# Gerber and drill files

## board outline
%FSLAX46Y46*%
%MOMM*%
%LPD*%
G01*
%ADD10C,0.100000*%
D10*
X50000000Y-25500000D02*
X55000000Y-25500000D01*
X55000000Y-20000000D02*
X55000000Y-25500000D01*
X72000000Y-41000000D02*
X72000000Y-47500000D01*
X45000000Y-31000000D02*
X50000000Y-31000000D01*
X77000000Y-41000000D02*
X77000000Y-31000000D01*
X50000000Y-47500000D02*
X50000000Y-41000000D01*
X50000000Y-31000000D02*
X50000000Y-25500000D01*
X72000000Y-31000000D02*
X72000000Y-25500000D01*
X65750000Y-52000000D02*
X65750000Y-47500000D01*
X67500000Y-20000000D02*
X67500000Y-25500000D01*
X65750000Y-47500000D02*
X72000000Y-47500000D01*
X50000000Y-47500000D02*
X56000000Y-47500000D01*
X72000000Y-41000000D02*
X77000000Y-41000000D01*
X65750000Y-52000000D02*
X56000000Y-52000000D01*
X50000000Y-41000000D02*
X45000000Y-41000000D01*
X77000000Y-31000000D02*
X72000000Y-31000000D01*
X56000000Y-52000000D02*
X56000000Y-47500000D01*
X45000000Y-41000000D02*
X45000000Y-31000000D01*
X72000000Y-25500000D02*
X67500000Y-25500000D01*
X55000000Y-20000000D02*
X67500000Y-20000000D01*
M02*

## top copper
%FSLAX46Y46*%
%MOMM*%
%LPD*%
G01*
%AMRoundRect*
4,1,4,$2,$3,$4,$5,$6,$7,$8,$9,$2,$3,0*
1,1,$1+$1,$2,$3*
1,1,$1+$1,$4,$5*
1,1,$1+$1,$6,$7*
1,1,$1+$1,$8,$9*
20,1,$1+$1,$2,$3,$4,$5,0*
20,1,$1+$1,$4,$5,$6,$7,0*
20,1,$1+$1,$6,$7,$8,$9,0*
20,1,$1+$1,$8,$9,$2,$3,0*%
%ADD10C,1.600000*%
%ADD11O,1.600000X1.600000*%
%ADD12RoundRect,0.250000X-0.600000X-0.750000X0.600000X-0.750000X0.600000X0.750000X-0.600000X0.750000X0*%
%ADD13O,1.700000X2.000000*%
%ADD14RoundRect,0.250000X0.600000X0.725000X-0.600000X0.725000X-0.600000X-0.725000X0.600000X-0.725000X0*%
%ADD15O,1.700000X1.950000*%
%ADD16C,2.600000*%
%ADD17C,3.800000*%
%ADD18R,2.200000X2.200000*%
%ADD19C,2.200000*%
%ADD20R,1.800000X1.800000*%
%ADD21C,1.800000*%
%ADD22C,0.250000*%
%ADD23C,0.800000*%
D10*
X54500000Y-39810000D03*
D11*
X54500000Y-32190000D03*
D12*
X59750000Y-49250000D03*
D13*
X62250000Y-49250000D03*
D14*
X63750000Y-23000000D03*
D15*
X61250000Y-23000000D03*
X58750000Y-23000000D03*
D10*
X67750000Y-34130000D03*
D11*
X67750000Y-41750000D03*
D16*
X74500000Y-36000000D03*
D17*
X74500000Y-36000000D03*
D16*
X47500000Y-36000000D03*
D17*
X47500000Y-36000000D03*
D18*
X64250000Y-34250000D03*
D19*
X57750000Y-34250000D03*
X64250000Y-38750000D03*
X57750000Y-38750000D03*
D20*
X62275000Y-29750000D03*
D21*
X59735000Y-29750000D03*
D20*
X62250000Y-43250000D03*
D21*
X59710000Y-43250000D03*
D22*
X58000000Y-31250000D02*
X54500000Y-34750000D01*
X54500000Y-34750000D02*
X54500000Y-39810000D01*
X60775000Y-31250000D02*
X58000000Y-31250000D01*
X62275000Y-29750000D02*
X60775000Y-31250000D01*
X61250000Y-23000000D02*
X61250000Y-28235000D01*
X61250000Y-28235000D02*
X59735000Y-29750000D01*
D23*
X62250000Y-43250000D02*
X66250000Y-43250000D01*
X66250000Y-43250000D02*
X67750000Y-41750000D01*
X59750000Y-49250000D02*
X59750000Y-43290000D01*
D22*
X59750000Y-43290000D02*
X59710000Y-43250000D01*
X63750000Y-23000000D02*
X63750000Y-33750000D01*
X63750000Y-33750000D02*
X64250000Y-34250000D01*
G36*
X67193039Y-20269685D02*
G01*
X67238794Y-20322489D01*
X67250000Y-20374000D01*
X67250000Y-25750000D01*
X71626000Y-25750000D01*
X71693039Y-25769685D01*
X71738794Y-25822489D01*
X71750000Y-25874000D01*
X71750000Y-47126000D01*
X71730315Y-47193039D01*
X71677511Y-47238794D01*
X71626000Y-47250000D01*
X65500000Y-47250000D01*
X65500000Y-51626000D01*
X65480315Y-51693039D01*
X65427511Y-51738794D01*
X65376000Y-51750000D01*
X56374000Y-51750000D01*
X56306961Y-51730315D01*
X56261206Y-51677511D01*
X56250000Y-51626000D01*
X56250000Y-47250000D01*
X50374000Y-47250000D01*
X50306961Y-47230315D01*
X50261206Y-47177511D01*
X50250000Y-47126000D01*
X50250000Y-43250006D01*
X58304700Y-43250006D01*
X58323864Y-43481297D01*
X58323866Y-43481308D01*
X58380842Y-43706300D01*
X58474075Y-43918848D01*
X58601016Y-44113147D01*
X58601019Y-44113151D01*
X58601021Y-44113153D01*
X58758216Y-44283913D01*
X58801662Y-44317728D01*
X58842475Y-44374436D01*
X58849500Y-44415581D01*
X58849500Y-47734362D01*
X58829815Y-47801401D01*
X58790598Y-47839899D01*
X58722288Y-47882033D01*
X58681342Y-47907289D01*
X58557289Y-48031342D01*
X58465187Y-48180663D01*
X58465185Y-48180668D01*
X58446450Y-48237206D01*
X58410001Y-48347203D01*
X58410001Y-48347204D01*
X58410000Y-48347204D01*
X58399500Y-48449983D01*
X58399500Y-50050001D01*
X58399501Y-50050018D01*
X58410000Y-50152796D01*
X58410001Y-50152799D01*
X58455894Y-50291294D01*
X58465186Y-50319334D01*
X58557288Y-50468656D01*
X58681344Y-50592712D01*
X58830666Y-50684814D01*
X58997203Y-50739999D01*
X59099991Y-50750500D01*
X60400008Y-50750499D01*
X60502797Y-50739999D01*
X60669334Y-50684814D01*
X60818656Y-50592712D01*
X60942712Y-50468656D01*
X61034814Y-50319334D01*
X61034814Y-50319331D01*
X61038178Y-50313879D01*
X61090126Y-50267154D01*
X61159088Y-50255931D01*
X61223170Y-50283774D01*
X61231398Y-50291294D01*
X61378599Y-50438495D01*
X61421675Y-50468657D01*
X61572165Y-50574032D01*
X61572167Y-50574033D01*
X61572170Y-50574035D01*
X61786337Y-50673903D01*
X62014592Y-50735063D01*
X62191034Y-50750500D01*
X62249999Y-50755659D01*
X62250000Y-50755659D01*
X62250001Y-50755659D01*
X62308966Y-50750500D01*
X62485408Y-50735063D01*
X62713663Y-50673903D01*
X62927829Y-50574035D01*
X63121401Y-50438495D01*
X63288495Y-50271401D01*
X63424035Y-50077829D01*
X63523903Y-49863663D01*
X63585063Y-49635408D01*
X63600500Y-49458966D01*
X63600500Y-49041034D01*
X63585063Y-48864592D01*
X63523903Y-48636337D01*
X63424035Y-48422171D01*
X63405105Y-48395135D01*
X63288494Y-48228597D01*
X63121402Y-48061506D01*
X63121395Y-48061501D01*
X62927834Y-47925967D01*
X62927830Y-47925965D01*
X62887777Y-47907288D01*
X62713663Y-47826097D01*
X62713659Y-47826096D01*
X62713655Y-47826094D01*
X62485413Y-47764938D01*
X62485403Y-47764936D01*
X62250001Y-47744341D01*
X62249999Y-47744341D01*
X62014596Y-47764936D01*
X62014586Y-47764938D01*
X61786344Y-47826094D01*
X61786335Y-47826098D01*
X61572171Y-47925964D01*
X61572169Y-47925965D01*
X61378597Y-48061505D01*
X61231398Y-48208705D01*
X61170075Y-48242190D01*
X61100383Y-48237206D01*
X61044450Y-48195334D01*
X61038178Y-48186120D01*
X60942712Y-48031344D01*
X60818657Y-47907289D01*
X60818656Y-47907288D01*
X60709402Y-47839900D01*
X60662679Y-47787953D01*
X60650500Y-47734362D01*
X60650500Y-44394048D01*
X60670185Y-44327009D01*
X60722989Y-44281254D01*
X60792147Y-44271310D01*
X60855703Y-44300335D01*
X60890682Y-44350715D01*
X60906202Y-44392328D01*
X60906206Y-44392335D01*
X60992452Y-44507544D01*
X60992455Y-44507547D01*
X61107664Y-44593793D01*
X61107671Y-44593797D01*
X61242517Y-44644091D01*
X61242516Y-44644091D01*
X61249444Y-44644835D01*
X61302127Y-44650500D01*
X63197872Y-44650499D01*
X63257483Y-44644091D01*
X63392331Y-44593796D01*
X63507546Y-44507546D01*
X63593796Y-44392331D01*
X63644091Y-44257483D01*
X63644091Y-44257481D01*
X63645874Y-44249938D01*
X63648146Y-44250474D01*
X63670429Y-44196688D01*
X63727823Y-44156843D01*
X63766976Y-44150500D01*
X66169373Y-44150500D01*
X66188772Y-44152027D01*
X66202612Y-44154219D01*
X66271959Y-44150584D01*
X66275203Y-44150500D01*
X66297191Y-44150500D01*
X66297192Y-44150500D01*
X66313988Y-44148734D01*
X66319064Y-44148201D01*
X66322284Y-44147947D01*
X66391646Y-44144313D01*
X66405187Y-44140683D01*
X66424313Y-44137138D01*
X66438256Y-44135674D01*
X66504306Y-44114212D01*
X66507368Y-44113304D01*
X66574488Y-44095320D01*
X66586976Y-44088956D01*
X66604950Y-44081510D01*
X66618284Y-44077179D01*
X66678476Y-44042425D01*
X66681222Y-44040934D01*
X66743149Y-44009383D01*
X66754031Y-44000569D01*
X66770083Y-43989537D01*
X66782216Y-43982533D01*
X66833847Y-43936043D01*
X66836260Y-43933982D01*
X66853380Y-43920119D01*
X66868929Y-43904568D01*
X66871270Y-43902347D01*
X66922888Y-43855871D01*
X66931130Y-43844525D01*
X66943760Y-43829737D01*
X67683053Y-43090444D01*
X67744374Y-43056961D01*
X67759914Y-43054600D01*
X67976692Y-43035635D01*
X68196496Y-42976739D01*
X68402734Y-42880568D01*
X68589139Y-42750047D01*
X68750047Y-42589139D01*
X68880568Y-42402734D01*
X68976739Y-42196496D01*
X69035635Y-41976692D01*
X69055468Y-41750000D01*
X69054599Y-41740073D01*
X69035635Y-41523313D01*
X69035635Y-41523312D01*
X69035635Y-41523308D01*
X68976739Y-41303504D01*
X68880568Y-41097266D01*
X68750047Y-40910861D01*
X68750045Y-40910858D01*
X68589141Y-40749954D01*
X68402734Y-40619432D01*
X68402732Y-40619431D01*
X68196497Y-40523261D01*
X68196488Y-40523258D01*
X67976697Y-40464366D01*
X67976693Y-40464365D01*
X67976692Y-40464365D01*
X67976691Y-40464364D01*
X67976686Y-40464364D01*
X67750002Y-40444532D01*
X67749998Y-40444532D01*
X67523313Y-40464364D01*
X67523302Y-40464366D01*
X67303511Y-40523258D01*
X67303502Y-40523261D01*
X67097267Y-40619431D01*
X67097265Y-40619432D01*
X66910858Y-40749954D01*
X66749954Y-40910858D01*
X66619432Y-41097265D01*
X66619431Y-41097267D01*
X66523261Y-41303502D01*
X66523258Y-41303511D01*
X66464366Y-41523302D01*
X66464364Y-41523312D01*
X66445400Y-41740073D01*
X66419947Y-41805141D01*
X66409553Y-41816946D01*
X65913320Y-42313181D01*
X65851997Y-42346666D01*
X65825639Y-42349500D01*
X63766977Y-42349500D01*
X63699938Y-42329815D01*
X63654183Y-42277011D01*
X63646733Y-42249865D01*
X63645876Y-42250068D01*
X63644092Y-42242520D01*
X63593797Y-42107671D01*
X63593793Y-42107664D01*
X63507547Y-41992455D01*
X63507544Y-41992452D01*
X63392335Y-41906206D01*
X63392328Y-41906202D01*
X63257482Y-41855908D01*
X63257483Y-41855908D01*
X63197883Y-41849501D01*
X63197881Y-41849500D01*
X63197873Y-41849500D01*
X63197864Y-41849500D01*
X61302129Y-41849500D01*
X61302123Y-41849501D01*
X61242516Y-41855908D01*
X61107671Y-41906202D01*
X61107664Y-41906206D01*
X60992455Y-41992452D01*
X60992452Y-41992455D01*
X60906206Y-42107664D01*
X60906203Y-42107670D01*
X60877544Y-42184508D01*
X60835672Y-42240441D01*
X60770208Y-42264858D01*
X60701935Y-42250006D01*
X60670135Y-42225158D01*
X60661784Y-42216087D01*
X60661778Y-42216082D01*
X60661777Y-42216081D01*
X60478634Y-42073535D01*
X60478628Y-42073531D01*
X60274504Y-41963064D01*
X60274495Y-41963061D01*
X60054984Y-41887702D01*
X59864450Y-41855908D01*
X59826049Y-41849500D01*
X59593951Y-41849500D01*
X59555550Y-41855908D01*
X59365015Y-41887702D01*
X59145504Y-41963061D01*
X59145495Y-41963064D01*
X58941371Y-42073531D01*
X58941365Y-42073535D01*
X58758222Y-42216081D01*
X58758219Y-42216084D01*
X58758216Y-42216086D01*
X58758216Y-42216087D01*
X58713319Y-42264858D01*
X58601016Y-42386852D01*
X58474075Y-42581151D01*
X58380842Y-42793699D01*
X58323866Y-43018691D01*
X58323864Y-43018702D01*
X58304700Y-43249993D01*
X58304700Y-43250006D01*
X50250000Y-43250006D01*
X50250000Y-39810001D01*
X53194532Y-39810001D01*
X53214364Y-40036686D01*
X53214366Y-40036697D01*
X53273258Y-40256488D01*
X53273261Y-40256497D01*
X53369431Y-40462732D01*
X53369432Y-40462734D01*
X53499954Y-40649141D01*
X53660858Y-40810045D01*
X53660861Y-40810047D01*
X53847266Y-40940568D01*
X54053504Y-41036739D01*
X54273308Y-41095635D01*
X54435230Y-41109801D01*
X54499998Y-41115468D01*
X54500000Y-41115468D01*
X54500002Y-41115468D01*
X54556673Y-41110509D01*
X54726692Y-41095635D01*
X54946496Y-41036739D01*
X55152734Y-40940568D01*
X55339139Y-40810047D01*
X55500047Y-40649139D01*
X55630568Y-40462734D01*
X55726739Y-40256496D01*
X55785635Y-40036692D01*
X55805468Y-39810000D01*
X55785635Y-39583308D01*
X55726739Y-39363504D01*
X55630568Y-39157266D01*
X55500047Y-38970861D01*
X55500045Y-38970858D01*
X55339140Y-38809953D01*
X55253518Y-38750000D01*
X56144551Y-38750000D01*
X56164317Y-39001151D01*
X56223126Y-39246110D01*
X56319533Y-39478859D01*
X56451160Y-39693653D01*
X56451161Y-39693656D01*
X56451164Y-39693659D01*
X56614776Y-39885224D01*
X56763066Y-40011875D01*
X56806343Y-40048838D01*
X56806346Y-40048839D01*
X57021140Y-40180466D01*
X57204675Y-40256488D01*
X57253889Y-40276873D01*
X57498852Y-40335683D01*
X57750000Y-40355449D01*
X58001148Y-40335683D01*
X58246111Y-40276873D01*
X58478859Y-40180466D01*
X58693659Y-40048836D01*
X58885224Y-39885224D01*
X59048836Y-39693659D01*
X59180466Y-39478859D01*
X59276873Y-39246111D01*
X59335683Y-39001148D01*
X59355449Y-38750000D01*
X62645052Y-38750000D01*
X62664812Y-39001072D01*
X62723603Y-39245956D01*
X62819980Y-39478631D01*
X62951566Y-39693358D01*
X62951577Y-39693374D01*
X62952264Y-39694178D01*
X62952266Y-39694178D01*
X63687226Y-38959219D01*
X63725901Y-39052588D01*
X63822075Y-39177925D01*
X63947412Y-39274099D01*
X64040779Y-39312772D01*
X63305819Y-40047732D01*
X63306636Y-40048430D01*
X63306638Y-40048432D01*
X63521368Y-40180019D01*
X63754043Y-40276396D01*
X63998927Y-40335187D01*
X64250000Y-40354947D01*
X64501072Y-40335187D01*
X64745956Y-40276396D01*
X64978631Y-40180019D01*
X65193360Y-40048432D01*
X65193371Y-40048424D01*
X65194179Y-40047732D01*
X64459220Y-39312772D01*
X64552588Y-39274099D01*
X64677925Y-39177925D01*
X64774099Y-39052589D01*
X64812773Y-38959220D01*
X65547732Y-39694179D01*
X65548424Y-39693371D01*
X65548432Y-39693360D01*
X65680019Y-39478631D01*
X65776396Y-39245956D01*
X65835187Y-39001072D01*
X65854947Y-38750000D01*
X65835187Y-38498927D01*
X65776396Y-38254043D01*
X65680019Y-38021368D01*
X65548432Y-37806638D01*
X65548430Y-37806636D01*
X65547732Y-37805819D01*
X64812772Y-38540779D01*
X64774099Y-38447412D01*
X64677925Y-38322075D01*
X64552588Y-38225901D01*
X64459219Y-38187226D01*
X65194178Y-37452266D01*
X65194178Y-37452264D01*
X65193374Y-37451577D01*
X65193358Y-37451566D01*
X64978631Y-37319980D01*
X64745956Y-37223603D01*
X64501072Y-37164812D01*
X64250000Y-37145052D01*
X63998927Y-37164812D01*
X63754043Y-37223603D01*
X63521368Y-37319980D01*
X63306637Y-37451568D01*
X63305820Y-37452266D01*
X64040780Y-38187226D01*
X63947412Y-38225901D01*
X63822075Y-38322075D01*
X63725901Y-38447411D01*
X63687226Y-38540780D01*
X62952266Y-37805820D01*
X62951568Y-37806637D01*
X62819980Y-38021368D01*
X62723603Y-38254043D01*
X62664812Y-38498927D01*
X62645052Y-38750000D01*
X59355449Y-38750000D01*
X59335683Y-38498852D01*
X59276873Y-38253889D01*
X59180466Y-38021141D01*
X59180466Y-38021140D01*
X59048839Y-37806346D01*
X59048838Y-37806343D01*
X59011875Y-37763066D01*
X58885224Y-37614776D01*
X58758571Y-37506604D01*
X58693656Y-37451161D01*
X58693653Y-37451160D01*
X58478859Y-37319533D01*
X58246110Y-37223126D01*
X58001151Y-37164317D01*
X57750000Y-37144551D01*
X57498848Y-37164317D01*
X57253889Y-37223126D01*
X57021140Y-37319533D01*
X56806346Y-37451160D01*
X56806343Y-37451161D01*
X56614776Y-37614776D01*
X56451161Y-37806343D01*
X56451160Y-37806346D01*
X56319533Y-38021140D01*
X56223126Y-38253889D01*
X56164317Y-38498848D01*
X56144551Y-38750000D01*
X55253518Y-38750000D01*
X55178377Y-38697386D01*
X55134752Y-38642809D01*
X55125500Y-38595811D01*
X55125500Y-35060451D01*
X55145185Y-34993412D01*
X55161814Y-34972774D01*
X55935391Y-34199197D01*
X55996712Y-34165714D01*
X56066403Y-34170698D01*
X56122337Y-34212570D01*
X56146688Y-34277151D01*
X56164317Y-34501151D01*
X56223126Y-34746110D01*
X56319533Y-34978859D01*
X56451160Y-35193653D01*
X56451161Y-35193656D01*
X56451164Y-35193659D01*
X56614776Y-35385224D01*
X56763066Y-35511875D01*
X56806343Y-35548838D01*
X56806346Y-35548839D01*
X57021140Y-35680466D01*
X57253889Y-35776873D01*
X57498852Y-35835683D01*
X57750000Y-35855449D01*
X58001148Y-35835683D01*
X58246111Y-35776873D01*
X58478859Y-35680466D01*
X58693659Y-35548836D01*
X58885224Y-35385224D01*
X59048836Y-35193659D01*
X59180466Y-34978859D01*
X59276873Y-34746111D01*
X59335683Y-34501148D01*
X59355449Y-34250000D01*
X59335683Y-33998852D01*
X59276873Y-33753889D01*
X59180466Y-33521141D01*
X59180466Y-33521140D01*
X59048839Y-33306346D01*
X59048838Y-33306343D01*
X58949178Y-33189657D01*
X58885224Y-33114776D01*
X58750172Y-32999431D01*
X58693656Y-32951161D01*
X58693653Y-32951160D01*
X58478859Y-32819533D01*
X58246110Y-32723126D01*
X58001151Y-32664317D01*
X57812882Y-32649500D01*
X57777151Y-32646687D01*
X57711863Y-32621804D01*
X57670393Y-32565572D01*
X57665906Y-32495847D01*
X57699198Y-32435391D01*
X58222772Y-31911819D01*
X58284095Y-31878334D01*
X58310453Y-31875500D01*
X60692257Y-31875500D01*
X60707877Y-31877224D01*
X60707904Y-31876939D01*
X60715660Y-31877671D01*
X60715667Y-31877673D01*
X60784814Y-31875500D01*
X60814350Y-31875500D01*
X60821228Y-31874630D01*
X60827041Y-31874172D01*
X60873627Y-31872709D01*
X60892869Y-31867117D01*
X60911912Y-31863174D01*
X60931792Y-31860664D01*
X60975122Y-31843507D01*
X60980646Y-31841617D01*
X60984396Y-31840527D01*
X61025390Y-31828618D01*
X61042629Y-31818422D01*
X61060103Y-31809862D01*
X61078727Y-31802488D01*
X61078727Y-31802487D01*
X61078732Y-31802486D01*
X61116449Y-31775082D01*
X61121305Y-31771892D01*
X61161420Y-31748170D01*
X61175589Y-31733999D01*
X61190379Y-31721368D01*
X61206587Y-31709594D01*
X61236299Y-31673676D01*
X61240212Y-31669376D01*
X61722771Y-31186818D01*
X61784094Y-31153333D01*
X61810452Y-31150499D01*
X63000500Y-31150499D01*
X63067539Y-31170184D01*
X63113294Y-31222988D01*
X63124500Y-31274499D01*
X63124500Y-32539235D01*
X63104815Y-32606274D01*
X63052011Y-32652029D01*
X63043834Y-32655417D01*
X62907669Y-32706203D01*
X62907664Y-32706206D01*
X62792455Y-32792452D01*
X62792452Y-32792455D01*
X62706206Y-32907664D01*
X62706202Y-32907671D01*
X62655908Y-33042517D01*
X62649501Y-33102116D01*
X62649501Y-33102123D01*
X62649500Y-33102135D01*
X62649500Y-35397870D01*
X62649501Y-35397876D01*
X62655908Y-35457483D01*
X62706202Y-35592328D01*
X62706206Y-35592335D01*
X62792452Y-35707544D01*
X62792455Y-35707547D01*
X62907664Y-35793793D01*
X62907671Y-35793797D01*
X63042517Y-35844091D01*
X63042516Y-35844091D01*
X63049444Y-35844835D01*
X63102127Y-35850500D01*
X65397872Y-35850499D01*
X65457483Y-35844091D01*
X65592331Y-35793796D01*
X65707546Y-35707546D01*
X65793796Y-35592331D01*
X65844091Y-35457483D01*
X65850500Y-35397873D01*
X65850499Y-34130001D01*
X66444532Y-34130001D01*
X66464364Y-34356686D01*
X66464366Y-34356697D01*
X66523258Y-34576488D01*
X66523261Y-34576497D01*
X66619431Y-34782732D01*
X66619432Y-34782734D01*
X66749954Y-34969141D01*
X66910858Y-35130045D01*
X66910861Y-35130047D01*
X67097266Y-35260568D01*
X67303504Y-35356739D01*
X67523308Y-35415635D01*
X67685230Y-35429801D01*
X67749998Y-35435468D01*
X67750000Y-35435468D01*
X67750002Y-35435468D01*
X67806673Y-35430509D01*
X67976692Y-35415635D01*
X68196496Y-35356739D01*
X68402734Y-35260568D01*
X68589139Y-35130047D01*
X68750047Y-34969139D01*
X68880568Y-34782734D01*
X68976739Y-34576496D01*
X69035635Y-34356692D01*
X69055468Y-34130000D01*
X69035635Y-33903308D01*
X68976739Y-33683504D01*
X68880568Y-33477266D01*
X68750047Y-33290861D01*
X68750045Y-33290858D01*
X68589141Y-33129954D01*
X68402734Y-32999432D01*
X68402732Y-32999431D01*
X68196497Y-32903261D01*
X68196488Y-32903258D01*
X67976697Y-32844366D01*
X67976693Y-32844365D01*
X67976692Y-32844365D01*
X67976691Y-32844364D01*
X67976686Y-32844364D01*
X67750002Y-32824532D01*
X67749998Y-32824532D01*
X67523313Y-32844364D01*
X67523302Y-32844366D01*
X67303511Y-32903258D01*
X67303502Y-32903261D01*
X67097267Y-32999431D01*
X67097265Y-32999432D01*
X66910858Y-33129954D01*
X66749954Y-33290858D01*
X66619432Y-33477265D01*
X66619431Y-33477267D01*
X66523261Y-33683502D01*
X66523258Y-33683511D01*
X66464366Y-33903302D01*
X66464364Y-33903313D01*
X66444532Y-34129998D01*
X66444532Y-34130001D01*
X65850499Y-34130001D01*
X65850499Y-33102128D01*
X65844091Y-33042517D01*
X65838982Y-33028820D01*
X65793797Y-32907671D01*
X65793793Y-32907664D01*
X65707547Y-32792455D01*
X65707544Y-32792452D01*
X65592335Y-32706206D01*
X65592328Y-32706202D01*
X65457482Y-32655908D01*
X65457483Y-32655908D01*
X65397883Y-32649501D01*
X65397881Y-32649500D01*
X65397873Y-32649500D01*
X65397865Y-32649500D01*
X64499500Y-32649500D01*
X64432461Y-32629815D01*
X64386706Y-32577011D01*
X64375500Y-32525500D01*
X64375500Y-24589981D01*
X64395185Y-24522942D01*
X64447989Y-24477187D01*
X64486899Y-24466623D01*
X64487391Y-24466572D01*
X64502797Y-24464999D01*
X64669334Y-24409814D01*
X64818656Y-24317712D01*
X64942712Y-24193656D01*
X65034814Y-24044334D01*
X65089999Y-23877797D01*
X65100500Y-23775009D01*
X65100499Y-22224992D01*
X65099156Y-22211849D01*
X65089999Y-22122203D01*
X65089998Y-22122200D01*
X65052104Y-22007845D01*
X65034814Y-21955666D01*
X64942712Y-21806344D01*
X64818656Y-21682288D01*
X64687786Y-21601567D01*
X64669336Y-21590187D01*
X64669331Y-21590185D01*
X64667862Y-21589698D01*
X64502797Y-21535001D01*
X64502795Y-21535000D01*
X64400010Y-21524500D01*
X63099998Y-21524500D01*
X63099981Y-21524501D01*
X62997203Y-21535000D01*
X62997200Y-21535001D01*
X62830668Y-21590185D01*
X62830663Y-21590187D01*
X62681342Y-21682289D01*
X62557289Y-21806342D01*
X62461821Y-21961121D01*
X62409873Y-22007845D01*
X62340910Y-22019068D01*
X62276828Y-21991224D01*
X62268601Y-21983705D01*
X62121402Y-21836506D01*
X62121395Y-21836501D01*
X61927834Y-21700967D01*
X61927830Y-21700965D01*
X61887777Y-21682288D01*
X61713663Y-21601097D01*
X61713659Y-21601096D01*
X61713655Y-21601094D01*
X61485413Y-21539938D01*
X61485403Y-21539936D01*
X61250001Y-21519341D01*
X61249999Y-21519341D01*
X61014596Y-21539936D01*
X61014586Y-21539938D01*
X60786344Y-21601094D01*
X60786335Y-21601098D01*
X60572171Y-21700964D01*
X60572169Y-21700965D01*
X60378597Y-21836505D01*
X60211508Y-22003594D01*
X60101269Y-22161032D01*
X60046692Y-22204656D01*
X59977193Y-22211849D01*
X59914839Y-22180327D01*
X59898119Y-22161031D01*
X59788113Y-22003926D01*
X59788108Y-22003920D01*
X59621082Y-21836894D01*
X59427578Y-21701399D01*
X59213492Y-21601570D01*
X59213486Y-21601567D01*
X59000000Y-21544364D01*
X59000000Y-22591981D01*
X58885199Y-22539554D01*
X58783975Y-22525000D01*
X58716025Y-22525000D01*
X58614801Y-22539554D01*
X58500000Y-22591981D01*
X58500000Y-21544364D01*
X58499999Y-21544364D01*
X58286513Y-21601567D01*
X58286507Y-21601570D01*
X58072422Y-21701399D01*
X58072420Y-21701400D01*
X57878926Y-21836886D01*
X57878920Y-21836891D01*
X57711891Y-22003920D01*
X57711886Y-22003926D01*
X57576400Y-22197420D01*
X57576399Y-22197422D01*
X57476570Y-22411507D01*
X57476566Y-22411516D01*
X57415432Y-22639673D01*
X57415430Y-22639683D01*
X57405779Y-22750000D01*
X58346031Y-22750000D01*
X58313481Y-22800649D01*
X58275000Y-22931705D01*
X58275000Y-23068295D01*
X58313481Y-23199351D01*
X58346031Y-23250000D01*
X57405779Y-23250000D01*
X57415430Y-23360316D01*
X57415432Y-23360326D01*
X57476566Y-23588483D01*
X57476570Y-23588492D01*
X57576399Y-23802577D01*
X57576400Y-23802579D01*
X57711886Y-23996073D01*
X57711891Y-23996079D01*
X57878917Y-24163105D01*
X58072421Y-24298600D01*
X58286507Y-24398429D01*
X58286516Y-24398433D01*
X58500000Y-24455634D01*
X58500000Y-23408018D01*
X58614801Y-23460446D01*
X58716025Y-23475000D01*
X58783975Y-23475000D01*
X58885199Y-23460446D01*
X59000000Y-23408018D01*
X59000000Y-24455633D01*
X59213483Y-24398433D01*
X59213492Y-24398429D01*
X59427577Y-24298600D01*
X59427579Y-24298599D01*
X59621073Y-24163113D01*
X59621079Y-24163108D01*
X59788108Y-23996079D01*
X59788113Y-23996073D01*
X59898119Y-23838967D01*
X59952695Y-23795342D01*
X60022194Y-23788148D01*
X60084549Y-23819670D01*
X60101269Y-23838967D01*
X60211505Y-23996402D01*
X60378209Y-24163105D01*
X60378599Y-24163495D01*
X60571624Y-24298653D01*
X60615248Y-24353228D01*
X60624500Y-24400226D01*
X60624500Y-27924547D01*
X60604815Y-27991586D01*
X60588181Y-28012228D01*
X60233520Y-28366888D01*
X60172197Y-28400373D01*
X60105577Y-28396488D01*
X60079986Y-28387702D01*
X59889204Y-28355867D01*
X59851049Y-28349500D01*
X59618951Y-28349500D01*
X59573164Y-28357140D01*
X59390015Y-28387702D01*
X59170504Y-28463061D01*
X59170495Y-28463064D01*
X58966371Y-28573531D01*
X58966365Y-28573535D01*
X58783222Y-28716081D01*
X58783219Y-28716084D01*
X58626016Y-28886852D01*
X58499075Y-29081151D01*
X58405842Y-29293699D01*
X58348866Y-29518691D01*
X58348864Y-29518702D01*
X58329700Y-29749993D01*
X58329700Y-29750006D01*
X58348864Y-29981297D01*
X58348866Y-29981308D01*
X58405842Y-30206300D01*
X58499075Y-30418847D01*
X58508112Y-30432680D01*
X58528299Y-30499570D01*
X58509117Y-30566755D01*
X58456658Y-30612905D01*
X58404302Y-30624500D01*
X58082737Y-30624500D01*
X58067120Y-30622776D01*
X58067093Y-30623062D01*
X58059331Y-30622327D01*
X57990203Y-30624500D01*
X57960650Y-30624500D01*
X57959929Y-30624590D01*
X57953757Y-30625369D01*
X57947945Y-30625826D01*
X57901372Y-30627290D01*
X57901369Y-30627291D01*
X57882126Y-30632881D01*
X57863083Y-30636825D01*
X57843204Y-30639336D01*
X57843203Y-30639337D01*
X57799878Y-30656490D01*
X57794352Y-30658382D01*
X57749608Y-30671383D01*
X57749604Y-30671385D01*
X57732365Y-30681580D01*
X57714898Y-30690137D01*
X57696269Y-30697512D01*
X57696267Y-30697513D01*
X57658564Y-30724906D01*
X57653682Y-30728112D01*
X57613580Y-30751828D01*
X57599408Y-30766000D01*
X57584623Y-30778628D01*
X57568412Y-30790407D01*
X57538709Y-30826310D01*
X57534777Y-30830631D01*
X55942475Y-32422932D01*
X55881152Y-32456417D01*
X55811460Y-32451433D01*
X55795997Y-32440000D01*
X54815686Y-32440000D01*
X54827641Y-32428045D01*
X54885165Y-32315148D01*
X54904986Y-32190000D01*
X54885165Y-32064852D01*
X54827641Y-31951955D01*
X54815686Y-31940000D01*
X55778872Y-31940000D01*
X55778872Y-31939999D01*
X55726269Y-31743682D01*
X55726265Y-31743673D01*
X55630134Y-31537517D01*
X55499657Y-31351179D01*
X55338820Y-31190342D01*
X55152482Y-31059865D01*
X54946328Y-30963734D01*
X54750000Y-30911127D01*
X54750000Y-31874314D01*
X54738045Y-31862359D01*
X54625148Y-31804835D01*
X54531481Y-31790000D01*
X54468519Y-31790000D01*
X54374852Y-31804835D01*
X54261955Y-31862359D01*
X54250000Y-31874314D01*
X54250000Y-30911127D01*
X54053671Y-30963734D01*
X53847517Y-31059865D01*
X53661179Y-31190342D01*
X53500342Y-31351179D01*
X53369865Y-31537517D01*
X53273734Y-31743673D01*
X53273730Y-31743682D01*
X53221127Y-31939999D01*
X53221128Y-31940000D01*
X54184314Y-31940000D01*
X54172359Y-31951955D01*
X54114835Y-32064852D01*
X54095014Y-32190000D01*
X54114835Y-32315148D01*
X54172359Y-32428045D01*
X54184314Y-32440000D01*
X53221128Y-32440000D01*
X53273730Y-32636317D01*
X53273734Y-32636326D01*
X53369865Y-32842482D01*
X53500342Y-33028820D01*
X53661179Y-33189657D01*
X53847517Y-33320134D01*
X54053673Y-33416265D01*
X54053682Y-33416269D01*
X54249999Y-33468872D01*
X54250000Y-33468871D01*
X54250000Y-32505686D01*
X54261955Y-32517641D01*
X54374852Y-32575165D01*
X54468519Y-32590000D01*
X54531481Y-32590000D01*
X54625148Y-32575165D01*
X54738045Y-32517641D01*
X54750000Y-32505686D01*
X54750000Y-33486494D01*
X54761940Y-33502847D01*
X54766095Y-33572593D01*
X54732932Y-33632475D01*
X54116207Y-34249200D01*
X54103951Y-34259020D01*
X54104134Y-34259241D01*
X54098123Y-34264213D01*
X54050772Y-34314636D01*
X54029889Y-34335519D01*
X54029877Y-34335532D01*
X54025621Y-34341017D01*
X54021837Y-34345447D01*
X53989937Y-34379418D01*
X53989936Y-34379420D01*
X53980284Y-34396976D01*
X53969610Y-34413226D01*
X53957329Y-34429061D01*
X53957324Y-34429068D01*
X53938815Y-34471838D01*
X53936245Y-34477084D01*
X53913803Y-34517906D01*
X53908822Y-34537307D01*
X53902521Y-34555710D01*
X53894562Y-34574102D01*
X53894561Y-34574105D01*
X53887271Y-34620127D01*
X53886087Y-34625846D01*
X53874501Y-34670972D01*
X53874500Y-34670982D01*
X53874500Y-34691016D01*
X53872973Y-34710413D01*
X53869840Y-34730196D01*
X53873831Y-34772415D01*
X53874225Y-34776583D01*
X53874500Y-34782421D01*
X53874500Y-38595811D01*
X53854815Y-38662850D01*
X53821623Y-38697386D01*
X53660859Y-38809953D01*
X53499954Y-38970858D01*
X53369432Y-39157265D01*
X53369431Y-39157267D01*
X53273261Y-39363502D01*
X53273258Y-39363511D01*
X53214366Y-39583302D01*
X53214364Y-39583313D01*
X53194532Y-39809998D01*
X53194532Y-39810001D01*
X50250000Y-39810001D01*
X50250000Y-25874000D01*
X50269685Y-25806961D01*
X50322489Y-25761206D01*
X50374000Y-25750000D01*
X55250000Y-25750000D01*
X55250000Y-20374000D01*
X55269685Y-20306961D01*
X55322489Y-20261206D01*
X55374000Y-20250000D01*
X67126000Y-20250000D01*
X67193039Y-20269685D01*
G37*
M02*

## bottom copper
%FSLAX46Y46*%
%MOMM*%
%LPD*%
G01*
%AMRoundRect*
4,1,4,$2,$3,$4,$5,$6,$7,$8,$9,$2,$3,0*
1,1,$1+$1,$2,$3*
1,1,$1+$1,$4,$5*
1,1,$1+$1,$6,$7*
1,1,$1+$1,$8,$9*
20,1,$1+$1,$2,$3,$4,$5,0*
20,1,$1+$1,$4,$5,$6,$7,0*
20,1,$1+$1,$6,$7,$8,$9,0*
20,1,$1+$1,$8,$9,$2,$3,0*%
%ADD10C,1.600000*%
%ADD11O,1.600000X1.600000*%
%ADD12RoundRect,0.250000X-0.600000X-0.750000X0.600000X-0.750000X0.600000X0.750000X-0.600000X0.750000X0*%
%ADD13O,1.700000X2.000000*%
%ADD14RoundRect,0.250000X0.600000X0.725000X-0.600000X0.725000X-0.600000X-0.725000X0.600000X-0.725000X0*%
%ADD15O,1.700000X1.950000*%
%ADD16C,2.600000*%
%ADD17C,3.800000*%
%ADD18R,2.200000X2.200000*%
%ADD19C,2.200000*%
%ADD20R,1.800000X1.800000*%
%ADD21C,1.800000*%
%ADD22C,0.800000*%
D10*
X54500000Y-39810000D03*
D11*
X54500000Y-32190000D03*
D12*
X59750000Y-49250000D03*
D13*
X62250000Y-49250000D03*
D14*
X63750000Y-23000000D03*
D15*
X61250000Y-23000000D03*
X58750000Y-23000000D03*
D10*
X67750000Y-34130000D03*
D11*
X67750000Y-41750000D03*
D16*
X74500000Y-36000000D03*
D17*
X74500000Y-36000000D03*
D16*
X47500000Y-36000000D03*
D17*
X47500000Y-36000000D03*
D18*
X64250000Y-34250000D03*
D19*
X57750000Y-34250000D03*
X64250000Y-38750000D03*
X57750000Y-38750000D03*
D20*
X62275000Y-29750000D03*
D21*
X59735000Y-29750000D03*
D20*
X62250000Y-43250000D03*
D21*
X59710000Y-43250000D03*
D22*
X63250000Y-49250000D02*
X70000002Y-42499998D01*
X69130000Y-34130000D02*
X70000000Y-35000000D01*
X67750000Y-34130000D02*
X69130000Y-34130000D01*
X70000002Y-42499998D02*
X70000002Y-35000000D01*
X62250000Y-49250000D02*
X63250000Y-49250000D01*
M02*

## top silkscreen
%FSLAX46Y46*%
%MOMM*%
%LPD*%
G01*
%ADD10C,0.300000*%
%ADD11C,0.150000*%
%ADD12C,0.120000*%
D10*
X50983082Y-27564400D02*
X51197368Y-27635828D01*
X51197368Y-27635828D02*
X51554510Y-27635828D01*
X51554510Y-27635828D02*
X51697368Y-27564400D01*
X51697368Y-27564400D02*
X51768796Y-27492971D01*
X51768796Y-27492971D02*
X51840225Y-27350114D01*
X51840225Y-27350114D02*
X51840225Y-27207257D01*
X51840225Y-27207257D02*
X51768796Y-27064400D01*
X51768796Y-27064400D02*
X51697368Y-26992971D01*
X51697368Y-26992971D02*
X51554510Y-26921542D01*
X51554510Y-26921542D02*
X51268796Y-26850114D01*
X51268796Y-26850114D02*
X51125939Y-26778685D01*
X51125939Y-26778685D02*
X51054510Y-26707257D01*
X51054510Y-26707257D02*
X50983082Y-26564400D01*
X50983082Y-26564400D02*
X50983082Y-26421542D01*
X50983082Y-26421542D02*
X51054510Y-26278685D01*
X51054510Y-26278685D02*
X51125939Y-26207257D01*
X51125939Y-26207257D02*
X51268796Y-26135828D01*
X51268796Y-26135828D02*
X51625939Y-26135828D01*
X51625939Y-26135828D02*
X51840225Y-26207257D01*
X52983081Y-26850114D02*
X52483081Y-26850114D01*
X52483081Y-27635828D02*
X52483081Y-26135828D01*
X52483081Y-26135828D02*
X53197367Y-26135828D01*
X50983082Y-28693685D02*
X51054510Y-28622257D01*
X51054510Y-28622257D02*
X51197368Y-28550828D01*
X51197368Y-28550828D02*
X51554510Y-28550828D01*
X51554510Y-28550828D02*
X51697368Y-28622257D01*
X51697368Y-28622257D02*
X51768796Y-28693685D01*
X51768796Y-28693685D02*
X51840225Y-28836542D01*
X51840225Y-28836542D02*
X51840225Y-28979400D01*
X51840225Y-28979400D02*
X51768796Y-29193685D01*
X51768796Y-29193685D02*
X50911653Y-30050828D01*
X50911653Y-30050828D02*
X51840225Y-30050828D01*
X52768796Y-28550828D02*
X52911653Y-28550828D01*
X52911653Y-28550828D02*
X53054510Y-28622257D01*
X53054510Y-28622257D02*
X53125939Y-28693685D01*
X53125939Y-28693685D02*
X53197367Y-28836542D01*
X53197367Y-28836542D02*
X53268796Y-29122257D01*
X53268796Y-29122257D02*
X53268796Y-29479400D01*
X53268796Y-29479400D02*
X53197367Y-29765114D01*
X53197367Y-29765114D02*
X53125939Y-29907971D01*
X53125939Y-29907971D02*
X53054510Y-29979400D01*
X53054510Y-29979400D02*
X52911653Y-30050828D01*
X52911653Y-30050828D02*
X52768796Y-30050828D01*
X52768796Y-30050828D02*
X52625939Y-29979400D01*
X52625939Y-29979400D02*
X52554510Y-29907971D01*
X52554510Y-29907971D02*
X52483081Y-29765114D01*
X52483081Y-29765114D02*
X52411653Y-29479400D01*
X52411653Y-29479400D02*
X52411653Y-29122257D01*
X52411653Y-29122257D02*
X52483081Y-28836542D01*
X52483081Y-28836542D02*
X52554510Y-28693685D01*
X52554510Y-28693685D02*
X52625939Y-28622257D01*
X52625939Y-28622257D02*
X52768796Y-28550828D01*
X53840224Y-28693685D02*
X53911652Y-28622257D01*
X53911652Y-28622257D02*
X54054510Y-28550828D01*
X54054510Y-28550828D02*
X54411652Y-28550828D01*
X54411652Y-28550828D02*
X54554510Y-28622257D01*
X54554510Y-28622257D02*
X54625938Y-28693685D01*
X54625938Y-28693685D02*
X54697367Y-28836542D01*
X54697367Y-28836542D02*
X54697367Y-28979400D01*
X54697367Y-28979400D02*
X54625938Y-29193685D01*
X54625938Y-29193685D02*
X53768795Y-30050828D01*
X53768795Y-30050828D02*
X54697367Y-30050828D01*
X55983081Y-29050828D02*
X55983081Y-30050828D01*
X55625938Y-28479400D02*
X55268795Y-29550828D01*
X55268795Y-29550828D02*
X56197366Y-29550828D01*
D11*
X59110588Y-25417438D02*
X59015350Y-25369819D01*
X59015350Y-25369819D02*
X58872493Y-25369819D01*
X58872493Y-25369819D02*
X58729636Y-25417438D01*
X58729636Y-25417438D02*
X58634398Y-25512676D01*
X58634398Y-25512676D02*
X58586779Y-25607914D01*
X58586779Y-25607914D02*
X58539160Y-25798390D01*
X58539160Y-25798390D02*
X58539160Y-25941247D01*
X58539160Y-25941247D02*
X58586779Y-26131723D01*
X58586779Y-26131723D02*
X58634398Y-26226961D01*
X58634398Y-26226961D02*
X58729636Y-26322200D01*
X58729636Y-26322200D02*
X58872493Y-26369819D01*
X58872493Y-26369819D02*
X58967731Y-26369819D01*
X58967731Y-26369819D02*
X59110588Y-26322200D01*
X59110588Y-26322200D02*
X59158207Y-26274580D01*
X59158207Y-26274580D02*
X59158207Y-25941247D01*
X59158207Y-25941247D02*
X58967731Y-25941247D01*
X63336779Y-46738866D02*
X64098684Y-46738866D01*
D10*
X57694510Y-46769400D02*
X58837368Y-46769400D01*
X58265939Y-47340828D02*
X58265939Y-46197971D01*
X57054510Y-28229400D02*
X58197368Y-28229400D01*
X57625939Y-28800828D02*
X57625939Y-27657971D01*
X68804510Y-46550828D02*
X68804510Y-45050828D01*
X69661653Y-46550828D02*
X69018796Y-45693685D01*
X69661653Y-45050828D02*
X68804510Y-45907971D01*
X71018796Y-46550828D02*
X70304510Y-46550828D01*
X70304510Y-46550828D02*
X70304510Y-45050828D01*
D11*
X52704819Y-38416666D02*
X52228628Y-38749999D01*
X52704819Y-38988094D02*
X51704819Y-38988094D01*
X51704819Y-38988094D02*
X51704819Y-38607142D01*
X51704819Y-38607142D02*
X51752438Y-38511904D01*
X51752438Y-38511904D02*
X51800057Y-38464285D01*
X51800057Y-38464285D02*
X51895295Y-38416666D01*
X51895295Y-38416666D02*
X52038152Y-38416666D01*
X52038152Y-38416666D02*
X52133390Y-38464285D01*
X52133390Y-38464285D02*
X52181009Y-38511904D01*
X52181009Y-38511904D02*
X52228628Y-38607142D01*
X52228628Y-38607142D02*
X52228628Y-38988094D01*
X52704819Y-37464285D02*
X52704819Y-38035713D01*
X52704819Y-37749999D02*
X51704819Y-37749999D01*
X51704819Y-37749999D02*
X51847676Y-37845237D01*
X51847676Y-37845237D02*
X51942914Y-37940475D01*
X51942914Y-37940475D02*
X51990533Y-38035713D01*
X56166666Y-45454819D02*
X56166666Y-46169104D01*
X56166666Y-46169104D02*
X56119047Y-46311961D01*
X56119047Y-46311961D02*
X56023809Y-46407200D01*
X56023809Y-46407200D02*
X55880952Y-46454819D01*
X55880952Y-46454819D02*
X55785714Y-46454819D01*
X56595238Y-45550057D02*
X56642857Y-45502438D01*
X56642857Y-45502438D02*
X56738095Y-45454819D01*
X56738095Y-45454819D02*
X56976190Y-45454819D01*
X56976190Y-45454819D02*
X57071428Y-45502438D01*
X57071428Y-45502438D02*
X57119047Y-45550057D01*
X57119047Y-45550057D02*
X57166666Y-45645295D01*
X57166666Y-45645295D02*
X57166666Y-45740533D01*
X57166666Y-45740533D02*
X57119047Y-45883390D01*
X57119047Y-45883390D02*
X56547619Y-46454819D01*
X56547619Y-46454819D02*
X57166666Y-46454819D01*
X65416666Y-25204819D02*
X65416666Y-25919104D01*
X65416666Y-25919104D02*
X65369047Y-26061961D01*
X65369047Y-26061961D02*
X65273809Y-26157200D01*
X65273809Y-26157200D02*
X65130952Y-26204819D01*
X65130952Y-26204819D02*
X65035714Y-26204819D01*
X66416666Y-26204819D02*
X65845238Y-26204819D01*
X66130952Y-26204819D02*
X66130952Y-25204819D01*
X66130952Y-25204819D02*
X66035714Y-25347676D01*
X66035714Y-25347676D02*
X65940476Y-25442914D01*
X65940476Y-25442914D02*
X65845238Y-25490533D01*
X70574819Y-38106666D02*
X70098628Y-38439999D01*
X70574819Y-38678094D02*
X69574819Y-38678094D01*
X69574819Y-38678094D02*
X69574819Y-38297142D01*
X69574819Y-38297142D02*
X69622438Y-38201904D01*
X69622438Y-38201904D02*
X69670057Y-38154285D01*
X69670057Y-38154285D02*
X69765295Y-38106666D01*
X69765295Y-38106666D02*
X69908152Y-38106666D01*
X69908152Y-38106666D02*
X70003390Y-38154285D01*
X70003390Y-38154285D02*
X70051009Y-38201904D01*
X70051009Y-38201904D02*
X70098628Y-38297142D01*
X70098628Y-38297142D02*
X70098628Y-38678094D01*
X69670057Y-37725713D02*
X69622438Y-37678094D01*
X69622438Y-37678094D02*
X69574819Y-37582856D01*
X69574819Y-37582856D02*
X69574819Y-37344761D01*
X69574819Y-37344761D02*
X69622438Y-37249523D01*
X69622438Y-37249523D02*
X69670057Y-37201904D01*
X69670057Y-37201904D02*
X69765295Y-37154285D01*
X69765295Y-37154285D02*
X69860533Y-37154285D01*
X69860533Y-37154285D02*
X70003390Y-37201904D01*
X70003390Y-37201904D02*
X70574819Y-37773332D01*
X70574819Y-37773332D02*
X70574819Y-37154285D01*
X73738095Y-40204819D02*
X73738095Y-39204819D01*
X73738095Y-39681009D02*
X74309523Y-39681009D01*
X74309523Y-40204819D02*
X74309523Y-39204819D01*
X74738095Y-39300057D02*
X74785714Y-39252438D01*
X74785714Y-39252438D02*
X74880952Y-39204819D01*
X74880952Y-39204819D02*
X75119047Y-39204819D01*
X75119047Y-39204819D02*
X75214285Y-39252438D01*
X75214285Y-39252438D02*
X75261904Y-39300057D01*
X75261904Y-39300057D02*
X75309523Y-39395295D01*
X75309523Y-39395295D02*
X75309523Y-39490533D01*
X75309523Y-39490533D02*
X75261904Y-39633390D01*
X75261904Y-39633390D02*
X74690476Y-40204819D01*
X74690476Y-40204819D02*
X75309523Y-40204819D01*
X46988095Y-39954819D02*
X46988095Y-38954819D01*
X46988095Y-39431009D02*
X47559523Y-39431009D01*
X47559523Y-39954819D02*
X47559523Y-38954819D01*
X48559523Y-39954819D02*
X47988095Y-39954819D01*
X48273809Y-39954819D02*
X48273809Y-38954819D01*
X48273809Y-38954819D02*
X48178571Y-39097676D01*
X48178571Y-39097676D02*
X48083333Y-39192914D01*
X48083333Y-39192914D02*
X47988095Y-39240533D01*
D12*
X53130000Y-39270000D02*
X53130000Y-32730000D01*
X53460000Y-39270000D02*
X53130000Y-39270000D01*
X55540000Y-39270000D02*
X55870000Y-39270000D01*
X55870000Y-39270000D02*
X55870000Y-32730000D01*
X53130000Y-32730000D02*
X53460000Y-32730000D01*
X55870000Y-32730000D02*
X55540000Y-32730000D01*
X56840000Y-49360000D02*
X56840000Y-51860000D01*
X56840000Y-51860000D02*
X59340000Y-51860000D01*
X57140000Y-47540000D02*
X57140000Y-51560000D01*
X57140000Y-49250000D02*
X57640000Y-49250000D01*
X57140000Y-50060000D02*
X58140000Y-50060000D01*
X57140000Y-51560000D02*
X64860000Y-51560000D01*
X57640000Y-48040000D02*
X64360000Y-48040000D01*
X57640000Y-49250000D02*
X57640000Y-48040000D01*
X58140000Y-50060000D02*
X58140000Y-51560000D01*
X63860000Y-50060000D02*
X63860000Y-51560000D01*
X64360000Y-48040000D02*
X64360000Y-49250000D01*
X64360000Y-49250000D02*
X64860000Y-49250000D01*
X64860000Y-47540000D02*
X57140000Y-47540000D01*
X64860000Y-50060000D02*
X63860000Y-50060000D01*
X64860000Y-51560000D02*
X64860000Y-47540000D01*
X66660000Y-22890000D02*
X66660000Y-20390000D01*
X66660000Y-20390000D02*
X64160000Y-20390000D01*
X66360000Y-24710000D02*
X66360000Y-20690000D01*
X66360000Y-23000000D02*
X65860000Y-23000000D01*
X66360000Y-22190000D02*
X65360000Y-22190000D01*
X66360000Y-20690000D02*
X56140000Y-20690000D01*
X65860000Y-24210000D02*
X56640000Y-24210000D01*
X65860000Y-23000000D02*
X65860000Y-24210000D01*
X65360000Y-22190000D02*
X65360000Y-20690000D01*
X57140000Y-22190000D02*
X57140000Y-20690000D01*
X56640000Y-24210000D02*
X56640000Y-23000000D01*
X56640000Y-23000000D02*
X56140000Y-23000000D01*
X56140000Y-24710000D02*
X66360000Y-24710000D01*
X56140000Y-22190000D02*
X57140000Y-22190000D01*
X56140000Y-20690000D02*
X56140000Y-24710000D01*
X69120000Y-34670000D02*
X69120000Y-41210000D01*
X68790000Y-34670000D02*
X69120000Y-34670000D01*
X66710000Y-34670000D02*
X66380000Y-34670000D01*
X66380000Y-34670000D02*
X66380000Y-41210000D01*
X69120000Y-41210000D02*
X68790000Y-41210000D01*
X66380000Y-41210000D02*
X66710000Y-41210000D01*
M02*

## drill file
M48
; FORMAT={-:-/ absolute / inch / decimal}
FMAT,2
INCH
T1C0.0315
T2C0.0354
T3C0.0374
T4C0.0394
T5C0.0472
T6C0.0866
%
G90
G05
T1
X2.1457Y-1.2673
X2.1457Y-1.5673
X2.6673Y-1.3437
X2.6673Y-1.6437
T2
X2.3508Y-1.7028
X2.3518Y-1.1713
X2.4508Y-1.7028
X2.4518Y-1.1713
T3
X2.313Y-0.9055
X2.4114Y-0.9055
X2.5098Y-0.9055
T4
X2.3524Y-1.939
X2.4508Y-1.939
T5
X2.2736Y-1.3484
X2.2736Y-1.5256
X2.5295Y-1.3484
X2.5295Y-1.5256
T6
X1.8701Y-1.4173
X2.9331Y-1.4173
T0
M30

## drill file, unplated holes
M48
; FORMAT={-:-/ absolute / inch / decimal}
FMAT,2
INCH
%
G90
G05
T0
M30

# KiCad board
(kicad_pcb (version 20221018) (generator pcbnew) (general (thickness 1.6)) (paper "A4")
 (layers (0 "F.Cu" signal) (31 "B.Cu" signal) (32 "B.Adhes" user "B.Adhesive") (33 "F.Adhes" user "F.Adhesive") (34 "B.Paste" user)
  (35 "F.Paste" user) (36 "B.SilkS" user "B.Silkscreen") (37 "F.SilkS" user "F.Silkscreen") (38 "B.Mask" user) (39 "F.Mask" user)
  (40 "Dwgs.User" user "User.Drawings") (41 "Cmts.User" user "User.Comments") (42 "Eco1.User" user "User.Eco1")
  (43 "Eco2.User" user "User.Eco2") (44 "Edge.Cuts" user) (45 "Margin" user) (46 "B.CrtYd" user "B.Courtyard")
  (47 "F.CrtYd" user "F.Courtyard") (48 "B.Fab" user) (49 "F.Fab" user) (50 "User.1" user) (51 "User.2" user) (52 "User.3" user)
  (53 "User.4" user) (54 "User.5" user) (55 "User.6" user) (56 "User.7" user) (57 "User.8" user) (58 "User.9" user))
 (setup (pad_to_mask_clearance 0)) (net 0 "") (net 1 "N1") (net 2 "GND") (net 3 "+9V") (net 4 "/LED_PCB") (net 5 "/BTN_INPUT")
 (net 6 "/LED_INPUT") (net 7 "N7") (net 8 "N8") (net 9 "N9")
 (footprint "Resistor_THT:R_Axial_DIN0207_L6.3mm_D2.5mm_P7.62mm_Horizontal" (layer "F.Cu") (at 54.5 39.81 90)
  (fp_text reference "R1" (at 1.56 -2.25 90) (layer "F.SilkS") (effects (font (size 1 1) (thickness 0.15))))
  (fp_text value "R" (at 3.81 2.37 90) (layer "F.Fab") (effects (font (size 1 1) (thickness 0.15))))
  (fp_line (start 0.54 -1.37) (end 7.08 -1.37) (stroke (width 0.12) (type solid)) (layer "F.SilkS"))
  (fp_line (start 0.54 -1.04) (end 0.54 -1.37) (stroke (width 0.12) (type solid)) (layer "F.SilkS"))
  (fp_line (start 0.54 1.04) (end 0.54 1.37) (stroke (width 0.12) (type solid)) (layer "F.SilkS"))
  (fp_line (start 0.54 1.37) (end 7.08 1.37) (stroke (width 0.12) (type solid)) (layer "F.SilkS"))
  (fp_line (start 7.08 -1.37) (end 7.08 -1.04) (stroke (width 0.12) (type solid)) (layer "F.SilkS"))
  (fp_line (start 7.08 1.37) (end 7.08 1.04) (stroke (width 0.12) (type solid)) (layer "F.SilkS"))
  (pad "1" thru_hole circle (at 0 0 90) (size 1.6 1.6) (drill 0.8) (layers "*.Cu" "*.Mask") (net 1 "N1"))
  (pad "2" thru_hole oval (at 7.62 0 90) (size 1.6 1.6) (drill 0.8) (layers "*.Cu" "*.Mask") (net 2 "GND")))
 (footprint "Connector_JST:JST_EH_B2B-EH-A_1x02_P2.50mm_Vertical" (layer "F.Cu") (at 59.75 49.25)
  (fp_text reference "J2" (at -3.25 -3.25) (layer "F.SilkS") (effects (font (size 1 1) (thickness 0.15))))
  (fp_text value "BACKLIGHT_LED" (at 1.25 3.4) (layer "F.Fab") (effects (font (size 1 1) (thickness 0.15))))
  (fp_line (start -2.91 0.11) (end -2.91 2.61) (stroke (width 0.12) (type solid)) (layer "F.SilkS"))
  (fp_line (start -2.91 2.61) (end -0.41 2.61) (stroke (width 0.12) (type solid)) (layer "F.SilkS"))
  (fp_line (start -2.61 -1.71) (end -2.61 2.31) (stroke (width 0.12) (type solid)) (layer "F.SilkS"))
  (fp_line (start -2.61 0) (end -2.11 0) (stroke (width 0.12) (type solid)) (layer "F.SilkS"))
  (fp_line (start -2.61 0.81) (end -1.61 0.81) (stroke (width 0.12) (type solid)) (layer "F.SilkS"))
  (fp_line (start -2.61 2.31) (end 5.11 2.31) (stroke (width 0.12) (type solid)) (layer "F.SilkS"))
  (fp_line (start -2.11 -1.21) (end 4.61 -1.21) (stroke (width 0.12) (type solid)) (layer "F.SilkS"))
  (fp_line (start -2.11 0) (end -2.11 -1.21) (stroke (width 0.12) (type solid)) (layer "F.SilkS"))
  (fp_line (start -1.61 0.81) (end -1.61 2.31) (stroke (width 0.12) (type solid)) (layer "F.SilkS"))
  (fp_line (start 4.11 0.81) (end 4.11 2.31) (stroke (width 0.12) (type solid)) (layer "F.SilkS"))
  (fp_line (start 4.61 -1.21) (end 4.61 0) (stroke (width 0.12) (type solid)) (layer "F.SilkS"))
  (fp_line (start 4.61 0) (end 5.11 0) (stroke (width 0.12) (type solid)) (layer "F.SilkS"))
  (fp_line (start 5.11 -1.71) (end -2.61 -1.71) (stroke (width 0.12) (type solid)) (layer "F.SilkS"))
  (fp_line (start 5.11 0.81) (end 4.11 0.81) (stroke (width 0.12) (type solid)) (layer "F.SilkS"))
  (fp_line (start 5.11 2.31) (end 5.11 -1.71) (stroke (width 0.12) (type solid)) (layer "F.SilkS"))
  (pad "1" thru_hole roundrect (at 0 0) (size 1.7 2) (drill 1) (layers "*.Cu" "*.Mask") (roundrect_rratio 0.1470588235) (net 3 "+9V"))
  (pad "2" thru_hole oval (at 2.5 0) (size 1.7 2) (drill 1) (layers "*.Cu" "*.Mask") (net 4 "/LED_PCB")))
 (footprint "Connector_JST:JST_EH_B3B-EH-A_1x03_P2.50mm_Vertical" (layer "F.Cu") (at 63.75 23 180)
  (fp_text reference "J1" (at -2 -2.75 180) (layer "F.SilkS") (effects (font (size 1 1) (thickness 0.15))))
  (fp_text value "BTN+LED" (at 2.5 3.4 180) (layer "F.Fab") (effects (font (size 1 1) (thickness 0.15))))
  (fp_line (start -2.91 0.11) (end -2.91 2.61) (stroke (width 0.12) (type solid)) (layer "F.SilkS"))
  (fp_line (start -2.91 2.61) (end -0.41 2.61) (stroke (width 0.12) (type solid)) (layer "F.SilkS"))
  (fp_line (start -2.61 -1.71) (end -2.61 2.31) (stroke (width 0.12) (type solid)) (layer "F.SilkS"))
  (fp_line (start -2.61 0) (end -2.11 0) (stroke (width 0.12) (type solid)) (layer "F.SilkS"))
  (fp_line (start -2.61 0.81) (end -1.61 0.81) (stroke (width 0.12) (type solid)) (layer "F.SilkS"))
  (fp_line (start -2.61 2.31) (end 7.61 2.31) (stroke (width 0.12) (type solid)) (layer "F.SilkS"))
  (fp_line (start -2.11 -1.21) (end 7.11 -1.21) (stroke (width 0.12) (type solid)) (layer "F.SilkS"))
  (fp_line (start -2.11 0) (end -2.11 -1.21) (stroke (width 0.12) (type solid)) (layer "F.SilkS"))
  (fp_line (start -1.61 0.81) (end -1.61 2.31) (stroke (width 0.12) (type solid)) (layer "F.SilkS"))
  (fp_line (start 6.61 0.81) (end 6.61 2.31) (stroke (width 0.12) (type solid)) (layer "F.SilkS"))
  (fp_line (start 7.11 -1.21) (end 7.11 0) (stroke (width 0.12) (type solid)) (layer "F.SilkS"))
  (fp_line (start 7.11 0) (end 7.61 0) (stroke (width 0.12) (type solid)) (layer "F.SilkS"))
  (fp_line (start 7.61 -1.71) (end -2.61 -1.71) (stroke (width 0.12) (type solid)) (layer "F.SilkS"))
  (fp_line (start 7.61 0.81) (end 6.61 0.81) (stroke (width 0.12) (type solid)) (layer "F.SilkS"))
  (fp_line (start 7.61 2.31) (end 7.61 -1.71) (stroke (width 0.12) (type solid)) (layer "F.SilkS"))
  (pad "1" thru_hole roundrect (at 0 0 180) (size 1.7 1.95) (drill 0.95) (layers "*.Cu" "*.Mask") (roundrect_rratio 0.1470588235)
   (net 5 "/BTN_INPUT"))
  (pad "2" thru_hole oval (at 2.5 0 180) (size 1.7 1.95) (drill 0.95) (layers "*.Cu" "*.Mask") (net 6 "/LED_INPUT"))
  (pad "3" thru_hole oval (at 5 0 180) (size 1.7 1.95) (drill 0.95) (layers "*.Cu" "*.Mask") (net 2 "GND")))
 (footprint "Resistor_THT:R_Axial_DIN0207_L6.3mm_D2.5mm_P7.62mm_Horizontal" (layer "F.Cu") (at 67.75 34.13 -90)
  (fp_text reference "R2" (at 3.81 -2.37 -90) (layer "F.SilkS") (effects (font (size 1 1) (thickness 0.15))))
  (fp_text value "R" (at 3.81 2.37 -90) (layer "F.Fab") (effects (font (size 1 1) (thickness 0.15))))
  (fp_line (start 0.54 -1.37) (end 7.08 -1.37) (stroke (width 0.12) (type solid)) (layer "F.SilkS"))
  (fp_line (start 0.54 -1.04) (end 0.54 -1.37) (stroke (width 0.12) (type solid)) (layer "F.SilkS"))
  (fp_line (start 0.54 1.04) (end 0.54 1.37) (stroke (width 0.12) (type solid)) (layer "F.SilkS"))
  (fp_line (start 0.54 1.37) (end 7.08 1.37) (stroke (width 0.12) (type solid)) (layer "F.SilkS"))
  (fp_line (start 7.08 -1.37) (end 7.08 -1.04) (stroke (width 0.12) (type solid)) (layer "F.SilkS"))
  (fp_line (start 7.08 1.37) (end 7.08 1.04) (stroke (width 0.12) (type solid)) (layer "F.SilkS"))
  (pad "1" thru_hole circle (at 0 0 270) (size 1.6 1.6) (drill 0.8) (layers "*.Cu" "*.Mask") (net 4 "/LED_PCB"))
  (pad "2" thru_hole oval (at 7.62 0 270) (size 1.6 1.6) (drill 0.8) (layers "*.Cu" "*.Mask") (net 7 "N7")))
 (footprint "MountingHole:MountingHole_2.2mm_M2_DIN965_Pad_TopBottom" (layer "F.Cu") (at 74.5 36 180)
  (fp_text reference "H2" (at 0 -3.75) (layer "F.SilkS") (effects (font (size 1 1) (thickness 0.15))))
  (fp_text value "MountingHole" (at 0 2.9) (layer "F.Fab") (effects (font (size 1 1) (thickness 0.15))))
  (pad "1" thru_hole circle (at 0 0 180) (size 2.6 2.6) (drill 2.2) (layers "*.Cu" "*.Mask"))
  (pad "1" connect circle (at 0 0 180) (size 3.8 3.8) (layers "F.Cu" "F.Mask"))
  (pad "1" connect circle (at 0 0 180) (size 3.8 3.8) (layers "B.Cu" "B.Mask")))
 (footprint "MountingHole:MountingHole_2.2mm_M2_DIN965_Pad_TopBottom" (layer "F.Cu") (at 47.5 36 180)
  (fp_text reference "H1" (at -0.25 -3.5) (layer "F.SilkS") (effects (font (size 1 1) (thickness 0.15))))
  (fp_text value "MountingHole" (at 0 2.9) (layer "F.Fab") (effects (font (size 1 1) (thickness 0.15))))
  (pad "1" thru_hole circle (at 0 0 180) (size 2.6 2.6) (drill 2.2) (layers "*.Cu" "*.Mask"))
  (pad "1" connect circle (at 0 0 180) (size 3.8 3.8) (layers "F.Cu" "F.Mask"))
  (pad "1" connect circle (at 0 0 180) (size 3.8 3.8) (layers "B.Cu" "B.Mask")))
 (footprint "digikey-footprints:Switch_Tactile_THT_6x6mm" (layer "B.Cu") (at 64.25 34.25 180)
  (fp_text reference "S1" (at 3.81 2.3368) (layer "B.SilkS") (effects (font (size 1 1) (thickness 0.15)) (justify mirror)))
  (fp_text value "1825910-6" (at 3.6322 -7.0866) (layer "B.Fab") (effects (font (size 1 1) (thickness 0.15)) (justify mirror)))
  (pad "1" thru_hole rect (at 0 0 180) (size 2.2 2.2) (drill 1.2) (layers "*.Cu" "*.Mask") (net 5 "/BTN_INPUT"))
  (pad "2" thru_hole circle (at 6.5 0 180) (size 2.2 2.2) (drill 1.2) (layers "*.Cu" "*.Mask") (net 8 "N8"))
  (pad "3" thru_hole circle (at 0 -4.5 180) (size 2.2 2.2) (drill 1.2) (layers "*.Cu" "*.Mask") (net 2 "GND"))
  (pad "4" thru_hole circle (at 6.5 -4.5 180) (size 2.2 2.2) (drill 1.2) (layers "*.Cu" "*.Mask") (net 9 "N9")))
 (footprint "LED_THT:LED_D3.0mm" (layer "B.Cu") (at 62.275 29.75 180)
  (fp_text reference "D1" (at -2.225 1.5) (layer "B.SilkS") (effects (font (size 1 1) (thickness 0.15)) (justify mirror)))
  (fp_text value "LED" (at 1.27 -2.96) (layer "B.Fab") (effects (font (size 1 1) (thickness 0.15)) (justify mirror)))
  (pad "1" thru_hole rect (at 0 0 180) (size 1.8 1.8) (drill 0.9) (layers "*.Cu" "*.Mask") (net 1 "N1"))
  (pad "2" thru_hole circle (at 2.54 0 180) (size 1.8 1.8) (drill 0.9) (layers "*.Cu" "*.Mask") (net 6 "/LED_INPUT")))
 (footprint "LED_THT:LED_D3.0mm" (layer "B.Cu") (at 62.25 43.25 180)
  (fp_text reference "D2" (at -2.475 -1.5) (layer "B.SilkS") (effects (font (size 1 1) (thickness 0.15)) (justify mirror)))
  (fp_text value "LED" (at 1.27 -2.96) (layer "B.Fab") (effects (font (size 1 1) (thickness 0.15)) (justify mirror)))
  (pad "1" thru_hole rect (at 0 0 180) (size 1.8 1.8) (drill 0.9) (layers "*.Cu" "*.Mask") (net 7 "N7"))
  (pad "2" thru_hole circle (at 2.54 0 180) (size 1.8 1.8) (drill 0.9) (layers "*.Cu" "*.Mask") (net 3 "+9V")))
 (gr_line (start 50 25.5) (end 55 25.5) (stroke (width 0.1) (type default)) (layer "Edge.Cuts"))
 (gr_line (start 55 20) (end 55 25.5) (stroke (width 0.1) (type default)) (layer "Edge.Cuts"))
 (gr_line (start 72 41) (end 72 47.5) (stroke (width 0.1) (type default)) (layer "Edge.Cuts"))
 (gr_line (start 45 31) (end 50 31) (stroke (width 0.1) (type default)) (layer "Edge.Cuts"))
 (gr_line (start 77 41) (end 77 31) (stroke (width 0.1) (type default)) (layer "Edge.Cuts"))
 (gr_line (start 50 47.5) (end 50 41) (stroke (width 0.1) (type default)) (layer "Edge.Cuts"))
 (gr_line (start 50 31) (end 50 25.5) (stroke (width 0.1) (type default)) (layer "Edge.Cuts"))
 (gr_line (start 72 31) (end 72 25.5) (stroke (width 0.1) (type default)) (layer "Edge.Cuts"))
 (gr_line (start 65.75 52) (end 65.75 47.5) (stroke (width 0.1) (type default)) (layer "Edge.Cuts"))
 (gr_line (start 67.5 20) (end 67.5 25.5) (stroke (width 0.1) (type default)) (layer "Edge.Cuts"))
 (gr_line (start 65.75 47.5) (end 72 47.5) (stroke (width 0.1) (type default)) (layer "Edge.Cuts"))
 (gr_line (start 50 47.5) (end 56 47.5) (stroke (width 0.1) (type default)) (layer "Edge.Cuts"))
 (gr_line (start 72 41) (end 77 41) (stroke (width 0.1) (type default)) (layer "Edge.Cuts"))
 (gr_line (start 65.75 52) (end 56 52) (stroke (width 0.1) (type default)) (layer "Edge.Cuts"))
 (gr_line (start 50 41) (end 45 41) (stroke (width 0.1) (type default)) (layer "Edge.Cuts"))
 (gr_line (start 77 31) (end 72 31) (stroke (width 0.1) (type default)) (layer "Edge.Cuts"))
 (gr_line (start 56 52) (end 56 47.5) (stroke (width 0.1) (type default)) (layer "Edge.Cuts"))
 (gr_line (start 45 41) (end 45 31) (stroke (width 0.1) (type default)) (layer "Edge.Cuts"))
 (gr_line (start 72 25.5) (end 67.5 25.5) (stroke (width 0.1) (type default)) (layer "Edge.Cuts"))
 (gr_line (start 55 20) (end 67.5 20) (stroke (width 0.1) (type default)) (layer "Edge.Cuts"))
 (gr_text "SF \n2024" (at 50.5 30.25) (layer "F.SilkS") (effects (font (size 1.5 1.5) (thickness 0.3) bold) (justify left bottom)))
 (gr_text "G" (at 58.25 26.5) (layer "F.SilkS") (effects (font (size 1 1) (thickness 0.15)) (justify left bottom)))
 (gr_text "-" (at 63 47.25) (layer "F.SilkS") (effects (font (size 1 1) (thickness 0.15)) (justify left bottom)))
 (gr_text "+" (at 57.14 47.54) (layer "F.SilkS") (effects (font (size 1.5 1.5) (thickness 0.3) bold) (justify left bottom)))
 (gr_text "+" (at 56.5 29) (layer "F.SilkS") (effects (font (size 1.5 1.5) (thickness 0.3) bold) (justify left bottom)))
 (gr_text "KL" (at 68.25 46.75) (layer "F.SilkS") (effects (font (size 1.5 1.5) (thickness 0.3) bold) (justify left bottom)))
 (segment (start 58 31.25) (end 54.5 34.75) (width 0.25) (layer "F.Cu") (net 1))
 (segment (start 54.5 34.75) (end 54.5 39.81) (width 0.25) (layer "F.Cu") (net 1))
 (segment (start 60.775 31.25) (end 58 31.25) (width 0.25) (layer "F.Cu") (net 1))
 (segment (start 62.275 29.75) (end 60.775 31.25) (width 0.25) (layer "F.Cu") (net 1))
 (segment (start 61.25 23) (end 61.25 28.235) (width 0.25) (layer "F.Cu") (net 6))
 (segment (start 61.25 28.235) (end 59.735 29.75) (width 0.25) (layer "F.Cu") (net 6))
 (segment (start 62.25 43.25) (end 66.25 43.25) (width 0.8) (layer "F.Cu") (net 7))
 (segment (start 66.25 43.25) (end 67.75 41.75) (width 0.8) (layer "F.Cu") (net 7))
 (segment (start 59.75 49.25) (end 59.75 43.29) (width 0.8) (layer "F.Cu") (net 3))
 (segment (start 59.75 43.29) (end 59.71 43.25) (width 0.25) (layer "F.Cu") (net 3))
 (segment (start 63.75 23) (end 63.75 33.75) (width 0.25) (layer "F.Cu") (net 5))
 (segment (start 63.75 33.75) (end 64.25 34.25) (width 0.25) (layer "F.Cu") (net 5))
 (segment (start 63.25 49.25) (end 70.000002 42.499998) (width 0.8) (layer "B.Cu") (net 4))
 (segment (start 69.13 34.13) (end 70 35) (width 0.8) (layer "B.Cu") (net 4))
 (segment (start 67.75 34.13) (end 69.13 34.13) (width 0.8) (layer "B.Cu") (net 4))
 (segment (start 70.000002 42.499998) (end 70.000002 35) (width 0.8) (layer "B.Cu") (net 4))
 (segment (start 62.25 49.25) (end 63.25 49.25) (width 0.8) (layer "B.Cu") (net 4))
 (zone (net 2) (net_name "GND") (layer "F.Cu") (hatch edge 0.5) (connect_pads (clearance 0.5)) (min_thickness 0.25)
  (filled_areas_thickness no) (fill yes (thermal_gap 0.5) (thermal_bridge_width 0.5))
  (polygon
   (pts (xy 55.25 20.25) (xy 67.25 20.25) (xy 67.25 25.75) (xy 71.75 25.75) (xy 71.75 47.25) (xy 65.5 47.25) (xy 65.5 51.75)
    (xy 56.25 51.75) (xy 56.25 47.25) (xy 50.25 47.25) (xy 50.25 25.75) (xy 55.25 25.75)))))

